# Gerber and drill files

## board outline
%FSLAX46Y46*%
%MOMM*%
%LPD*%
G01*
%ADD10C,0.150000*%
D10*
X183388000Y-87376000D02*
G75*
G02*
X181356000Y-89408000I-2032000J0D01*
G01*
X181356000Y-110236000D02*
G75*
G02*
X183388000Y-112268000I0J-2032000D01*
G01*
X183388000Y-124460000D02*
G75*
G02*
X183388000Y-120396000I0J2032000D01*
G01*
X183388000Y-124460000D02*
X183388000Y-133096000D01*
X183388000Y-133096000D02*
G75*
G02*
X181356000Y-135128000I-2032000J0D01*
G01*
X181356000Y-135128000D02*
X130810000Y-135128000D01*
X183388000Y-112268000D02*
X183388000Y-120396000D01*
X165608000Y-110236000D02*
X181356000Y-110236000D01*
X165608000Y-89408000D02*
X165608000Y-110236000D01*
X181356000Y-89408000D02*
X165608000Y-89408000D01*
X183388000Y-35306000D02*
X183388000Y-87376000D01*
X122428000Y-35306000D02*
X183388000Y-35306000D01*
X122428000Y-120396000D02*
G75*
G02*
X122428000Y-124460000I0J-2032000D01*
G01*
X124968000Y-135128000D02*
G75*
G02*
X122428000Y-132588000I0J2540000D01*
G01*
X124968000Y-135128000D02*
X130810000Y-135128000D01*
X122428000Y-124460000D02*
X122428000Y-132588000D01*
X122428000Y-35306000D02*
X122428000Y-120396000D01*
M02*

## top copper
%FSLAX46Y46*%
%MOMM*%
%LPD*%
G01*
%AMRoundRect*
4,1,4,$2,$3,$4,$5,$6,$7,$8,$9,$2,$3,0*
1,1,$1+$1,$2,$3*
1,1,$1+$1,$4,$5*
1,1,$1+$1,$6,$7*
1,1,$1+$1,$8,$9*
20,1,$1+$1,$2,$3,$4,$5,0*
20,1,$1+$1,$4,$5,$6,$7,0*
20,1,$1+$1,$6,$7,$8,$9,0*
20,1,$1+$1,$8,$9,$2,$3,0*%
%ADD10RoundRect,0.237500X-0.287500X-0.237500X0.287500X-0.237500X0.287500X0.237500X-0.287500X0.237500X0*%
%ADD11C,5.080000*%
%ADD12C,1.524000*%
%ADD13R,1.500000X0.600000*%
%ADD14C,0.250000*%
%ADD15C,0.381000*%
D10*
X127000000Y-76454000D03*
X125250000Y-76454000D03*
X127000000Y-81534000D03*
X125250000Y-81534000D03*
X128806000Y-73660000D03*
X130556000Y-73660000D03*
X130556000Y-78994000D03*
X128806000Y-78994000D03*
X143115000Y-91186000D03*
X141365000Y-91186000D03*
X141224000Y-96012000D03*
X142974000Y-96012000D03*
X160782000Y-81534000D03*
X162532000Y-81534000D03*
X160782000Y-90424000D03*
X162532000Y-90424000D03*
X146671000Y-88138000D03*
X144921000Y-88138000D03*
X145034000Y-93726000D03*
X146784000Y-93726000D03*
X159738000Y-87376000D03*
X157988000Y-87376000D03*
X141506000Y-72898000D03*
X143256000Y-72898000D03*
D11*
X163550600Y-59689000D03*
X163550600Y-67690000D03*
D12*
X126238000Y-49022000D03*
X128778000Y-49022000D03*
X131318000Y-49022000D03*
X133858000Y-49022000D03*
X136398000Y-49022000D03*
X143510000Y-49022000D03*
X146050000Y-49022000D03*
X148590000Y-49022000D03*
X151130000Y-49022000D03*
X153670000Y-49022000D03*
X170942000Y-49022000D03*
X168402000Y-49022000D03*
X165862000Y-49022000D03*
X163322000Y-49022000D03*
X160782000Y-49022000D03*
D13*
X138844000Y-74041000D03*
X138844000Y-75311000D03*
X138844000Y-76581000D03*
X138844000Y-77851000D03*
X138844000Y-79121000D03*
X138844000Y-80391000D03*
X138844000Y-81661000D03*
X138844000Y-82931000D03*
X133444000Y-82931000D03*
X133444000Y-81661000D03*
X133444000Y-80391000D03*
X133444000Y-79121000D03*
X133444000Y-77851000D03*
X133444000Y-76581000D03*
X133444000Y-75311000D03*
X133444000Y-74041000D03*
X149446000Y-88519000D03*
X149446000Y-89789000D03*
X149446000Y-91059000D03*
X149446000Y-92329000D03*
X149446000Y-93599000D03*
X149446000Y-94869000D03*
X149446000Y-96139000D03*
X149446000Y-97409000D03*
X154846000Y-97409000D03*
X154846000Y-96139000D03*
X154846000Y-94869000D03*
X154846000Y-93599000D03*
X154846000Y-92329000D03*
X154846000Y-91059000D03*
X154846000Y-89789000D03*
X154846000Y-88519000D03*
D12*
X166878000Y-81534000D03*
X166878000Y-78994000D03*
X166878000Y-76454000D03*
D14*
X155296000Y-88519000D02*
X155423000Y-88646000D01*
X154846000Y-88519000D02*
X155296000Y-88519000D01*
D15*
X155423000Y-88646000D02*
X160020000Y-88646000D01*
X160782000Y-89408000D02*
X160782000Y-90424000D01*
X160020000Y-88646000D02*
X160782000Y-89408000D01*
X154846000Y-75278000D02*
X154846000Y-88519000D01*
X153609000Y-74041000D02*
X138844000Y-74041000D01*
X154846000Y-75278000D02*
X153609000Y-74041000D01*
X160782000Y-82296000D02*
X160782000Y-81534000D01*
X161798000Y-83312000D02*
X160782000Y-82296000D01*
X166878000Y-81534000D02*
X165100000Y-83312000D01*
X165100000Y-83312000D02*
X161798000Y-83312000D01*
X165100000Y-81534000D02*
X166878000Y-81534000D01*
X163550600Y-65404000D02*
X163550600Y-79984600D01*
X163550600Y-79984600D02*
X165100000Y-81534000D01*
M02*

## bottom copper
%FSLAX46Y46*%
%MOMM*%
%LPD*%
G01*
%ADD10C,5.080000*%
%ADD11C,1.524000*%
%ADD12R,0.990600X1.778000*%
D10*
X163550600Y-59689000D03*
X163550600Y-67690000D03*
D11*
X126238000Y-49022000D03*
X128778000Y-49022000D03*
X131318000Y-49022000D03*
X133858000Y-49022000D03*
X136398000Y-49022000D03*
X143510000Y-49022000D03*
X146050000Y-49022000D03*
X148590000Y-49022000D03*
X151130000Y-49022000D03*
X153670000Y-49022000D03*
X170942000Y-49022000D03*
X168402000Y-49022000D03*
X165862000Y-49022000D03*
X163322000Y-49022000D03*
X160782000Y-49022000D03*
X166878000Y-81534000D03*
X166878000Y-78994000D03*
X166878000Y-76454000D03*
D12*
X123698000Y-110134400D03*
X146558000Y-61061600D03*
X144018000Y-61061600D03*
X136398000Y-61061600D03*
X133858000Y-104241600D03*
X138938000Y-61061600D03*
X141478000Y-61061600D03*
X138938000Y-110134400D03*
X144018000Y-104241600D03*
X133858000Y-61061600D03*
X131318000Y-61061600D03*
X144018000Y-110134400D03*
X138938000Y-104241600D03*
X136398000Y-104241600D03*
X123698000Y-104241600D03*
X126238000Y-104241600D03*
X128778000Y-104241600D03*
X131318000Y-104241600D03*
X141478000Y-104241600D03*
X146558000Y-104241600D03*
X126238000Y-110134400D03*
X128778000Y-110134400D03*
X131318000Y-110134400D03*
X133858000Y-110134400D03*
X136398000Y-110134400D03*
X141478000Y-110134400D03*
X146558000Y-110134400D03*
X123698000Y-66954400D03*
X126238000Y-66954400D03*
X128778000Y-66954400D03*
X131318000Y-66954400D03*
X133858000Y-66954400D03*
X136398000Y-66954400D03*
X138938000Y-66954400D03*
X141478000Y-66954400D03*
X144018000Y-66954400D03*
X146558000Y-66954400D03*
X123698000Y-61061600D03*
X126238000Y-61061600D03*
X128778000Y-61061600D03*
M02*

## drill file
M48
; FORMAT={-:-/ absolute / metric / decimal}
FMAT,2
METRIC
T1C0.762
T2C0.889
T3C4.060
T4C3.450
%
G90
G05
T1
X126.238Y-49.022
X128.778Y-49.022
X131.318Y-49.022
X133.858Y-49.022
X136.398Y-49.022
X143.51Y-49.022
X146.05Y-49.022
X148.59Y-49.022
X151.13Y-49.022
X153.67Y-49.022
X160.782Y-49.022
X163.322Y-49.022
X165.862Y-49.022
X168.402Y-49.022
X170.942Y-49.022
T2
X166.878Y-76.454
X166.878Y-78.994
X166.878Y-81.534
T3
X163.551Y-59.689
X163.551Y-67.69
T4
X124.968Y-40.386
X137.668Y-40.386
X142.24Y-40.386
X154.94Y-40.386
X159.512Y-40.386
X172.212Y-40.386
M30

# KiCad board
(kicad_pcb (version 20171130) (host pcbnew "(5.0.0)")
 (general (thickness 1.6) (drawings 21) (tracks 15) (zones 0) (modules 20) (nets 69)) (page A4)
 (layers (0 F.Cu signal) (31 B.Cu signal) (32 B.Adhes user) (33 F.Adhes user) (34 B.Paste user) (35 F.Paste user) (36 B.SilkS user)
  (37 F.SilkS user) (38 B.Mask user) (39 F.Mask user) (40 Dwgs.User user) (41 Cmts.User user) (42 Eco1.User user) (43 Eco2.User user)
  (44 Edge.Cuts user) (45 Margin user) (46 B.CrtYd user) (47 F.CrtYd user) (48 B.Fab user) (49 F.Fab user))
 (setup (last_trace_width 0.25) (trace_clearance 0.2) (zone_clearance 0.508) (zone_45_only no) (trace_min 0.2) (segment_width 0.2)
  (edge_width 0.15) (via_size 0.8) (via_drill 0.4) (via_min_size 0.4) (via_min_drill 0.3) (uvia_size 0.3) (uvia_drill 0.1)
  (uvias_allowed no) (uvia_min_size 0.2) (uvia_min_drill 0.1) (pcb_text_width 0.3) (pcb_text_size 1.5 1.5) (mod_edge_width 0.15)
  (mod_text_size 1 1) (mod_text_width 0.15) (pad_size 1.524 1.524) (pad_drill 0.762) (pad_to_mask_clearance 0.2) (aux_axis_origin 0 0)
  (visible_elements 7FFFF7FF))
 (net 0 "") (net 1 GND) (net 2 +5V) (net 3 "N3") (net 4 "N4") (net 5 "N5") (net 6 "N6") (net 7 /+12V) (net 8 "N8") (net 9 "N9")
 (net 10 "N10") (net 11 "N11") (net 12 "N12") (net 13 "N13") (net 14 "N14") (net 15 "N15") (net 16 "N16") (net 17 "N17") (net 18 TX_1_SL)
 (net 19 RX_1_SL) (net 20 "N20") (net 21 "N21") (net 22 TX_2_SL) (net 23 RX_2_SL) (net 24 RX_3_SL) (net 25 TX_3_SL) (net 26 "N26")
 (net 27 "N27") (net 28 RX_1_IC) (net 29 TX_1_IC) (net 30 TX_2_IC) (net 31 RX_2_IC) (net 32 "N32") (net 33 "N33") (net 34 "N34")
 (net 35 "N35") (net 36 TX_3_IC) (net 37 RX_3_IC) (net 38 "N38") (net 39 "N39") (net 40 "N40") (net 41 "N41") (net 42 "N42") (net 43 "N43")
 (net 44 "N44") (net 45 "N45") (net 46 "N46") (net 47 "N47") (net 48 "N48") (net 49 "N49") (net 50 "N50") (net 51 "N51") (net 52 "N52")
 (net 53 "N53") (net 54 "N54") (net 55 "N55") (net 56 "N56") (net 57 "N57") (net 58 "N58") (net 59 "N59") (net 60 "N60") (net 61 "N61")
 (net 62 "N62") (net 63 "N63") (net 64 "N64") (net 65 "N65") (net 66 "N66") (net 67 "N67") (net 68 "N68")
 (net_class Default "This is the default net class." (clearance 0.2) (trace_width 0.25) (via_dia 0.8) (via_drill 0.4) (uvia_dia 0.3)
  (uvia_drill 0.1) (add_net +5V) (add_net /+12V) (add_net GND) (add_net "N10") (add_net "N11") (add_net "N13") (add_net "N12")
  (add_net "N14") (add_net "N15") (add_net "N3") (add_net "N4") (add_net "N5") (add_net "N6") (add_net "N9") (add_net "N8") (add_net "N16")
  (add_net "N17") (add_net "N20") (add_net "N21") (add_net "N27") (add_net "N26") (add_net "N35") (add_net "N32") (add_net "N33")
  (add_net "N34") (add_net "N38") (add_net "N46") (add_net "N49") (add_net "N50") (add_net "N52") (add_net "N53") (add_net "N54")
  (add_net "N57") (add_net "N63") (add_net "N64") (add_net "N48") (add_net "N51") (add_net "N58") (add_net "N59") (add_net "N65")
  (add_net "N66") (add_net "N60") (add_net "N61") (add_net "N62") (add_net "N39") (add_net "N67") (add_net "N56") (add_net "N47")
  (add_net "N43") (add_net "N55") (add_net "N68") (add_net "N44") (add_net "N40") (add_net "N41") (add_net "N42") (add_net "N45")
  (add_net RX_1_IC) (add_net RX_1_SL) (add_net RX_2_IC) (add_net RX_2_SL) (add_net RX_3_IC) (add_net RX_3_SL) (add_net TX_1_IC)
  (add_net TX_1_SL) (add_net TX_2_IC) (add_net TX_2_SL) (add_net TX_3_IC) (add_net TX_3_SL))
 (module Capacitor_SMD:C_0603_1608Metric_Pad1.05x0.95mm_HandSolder (layer F.Cu) (at 126.125 76.454)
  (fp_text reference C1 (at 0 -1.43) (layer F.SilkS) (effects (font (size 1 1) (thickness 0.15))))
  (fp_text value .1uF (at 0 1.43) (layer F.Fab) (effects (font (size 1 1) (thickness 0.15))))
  (pad 2 smd roundrect (at 0.875 0) (size 1.05 0.95) (layers F.Cu F.Paste F.Mask) (roundrect_rratio 0.25) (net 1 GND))
  (pad 1 smd roundrect (at -0.875 0) (size 1.05 0.95) (layers F.Cu F.Paste F.Mask) (roundrect_rratio 0.25) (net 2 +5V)))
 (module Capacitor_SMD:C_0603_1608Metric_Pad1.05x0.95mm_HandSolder (layer F.Cu) (at 126.125 81.534)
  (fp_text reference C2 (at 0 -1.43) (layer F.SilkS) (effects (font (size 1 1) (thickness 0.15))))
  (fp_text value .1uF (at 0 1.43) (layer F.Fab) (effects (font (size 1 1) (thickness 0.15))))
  (pad 2 smd roundrect (at 0.875 0) (size 1.05 0.95) (layers F.Cu F.Paste F.Mask) (roundrect_rratio 0.25) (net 1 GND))
  (pad 1 smd roundrect (at -0.875 0) (size 1.05 0.95) (layers F.Cu F.Paste F.Mask) (roundrect_rratio 0.25) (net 2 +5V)))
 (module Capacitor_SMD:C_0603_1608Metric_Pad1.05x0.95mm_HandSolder (layer F.Cu) (at 129.681 73.66)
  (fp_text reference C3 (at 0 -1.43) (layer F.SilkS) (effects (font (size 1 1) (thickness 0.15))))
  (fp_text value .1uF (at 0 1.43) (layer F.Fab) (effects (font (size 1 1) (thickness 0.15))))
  (pad 1 smd roundrect (at -0.875 0) (size 1.05 0.95) (layers F.Cu F.Paste F.Mask) (roundrect_rratio 0.25) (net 1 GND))
  (pad 2 smd roundrect (at 0.875 0) (size 1.05 0.95) (layers F.Cu F.Paste F.Mask) (roundrect_rratio 0.25) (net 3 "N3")))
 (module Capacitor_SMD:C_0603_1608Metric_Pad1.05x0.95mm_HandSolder (layer F.Cu) (at 129.681 78.994)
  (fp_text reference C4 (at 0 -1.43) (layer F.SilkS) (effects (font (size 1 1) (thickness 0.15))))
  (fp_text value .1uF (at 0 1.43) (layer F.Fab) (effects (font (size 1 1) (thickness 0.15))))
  (pad 2 smd roundrect (at 0.875 0) (size 1.05 0.95) (layers F.Cu F.Paste F.Mask) (roundrect_rratio 0.25) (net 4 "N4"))
  (pad 1 smd roundrect (at -0.875 0) (size 1.05 0.95) (layers F.Cu F.Paste F.Mask) (roundrect_rratio 0.25) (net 1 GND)))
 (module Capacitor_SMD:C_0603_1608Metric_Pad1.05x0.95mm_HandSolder (layer F.Cu) (at 142.24 91.186)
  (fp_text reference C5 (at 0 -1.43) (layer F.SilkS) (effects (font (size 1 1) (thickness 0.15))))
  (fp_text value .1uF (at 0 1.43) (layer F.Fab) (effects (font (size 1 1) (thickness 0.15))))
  (pad 2 smd roundrect (at 0.875 0) (size 1.05 0.95) (layers F.Cu F.Paste F.Mask) (roundrect_rratio 0.25) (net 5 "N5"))
  (pad 1 smd roundrect (at -0.875 0) (size 1.05 0.95) (layers F.Cu F.Paste F.Mask) (roundrect_rratio 0.25) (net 1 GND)))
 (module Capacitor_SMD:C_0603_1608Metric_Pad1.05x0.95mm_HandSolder (layer F.Cu) (at 142.099 96.012)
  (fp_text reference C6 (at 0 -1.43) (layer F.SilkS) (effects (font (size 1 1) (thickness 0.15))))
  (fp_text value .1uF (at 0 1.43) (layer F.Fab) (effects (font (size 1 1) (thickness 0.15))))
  (pad 1 smd roundrect (at -0.875 0) (size 1.05 0.95) (layers F.Cu F.Paste F.Mask) (roundrect_rratio 0.25) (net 1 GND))
  (pad 2 smd roundrect (at 0.875 0) (size 1.05 0.95) (layers F.Cu F.Paste F.Mask) (roundrect_rratio 0.25) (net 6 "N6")))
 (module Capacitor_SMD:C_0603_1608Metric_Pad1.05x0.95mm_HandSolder (layer F.Cu) (at 161.657 81.534)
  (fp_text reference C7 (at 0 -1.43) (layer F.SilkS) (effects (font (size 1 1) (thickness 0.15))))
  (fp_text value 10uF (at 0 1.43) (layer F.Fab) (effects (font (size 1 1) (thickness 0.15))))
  (pad 1 smd roundrect (at -0.875 0) (size 1.05 0.95) (layers F.Cu F.Paste F.Mask) (roundrect_rratio 0.25) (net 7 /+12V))
  (pad 2 smd roundrect (at 0.875 0) (size 1.05 0.95) (layers F.Cu F.Paste F.Mask) (roundrect_rratio 0.25) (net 1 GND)))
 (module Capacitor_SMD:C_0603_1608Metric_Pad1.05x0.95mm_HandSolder (layer F.Cu) (at 161.657 90.424)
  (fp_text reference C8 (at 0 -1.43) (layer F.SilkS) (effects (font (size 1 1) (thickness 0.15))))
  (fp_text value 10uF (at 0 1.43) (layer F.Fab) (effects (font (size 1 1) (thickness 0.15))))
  (pad 1 smd roundrect (at -0.875 0) (size 1.05 0.95) (layers F.Cu F.Paste F.Mask) (roundrect_rratio 0.25) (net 2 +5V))
  (pad 2 smd roundrect (at 0.875 0) (size 1.05 0.95) (layers F.Cu F.Paste F.Mask) (roundrect_rratio 0.25) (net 1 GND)))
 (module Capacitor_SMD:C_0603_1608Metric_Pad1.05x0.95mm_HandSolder (layer F.Cu) (at 145.796 88.138)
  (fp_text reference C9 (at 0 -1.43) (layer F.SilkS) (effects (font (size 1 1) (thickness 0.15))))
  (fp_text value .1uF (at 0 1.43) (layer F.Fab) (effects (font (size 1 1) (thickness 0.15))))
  (pad 2 smd roundrect (at 0.875 0) (size 1.05 0.95) (layers F.Cu F.Paste F.Mask) (roundrect_rratio 0.25) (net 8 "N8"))
  (pad 1 smd roundrect (at -0.875 0) (size 1.05 0.95) (layers F.Cu F.Paste F.Mask) (roundrect_rratio 0.25) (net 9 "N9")))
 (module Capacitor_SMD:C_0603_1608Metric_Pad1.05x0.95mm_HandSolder (layer F.Cu) (at 145.909 93.726)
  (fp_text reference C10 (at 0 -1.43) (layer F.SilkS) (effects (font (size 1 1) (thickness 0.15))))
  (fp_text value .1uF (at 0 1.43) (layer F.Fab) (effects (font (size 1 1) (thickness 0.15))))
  (pad 1 smd roundrect (at -0.875 0) (size 1.05 0.95) (layers F.Cu F.Paste F.Mask) (roundrect_rratio 0.25) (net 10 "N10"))
  (pad 2 smd roundrect (at 0.875 0) (size 1.05 0.95) (layers F.Cu F.Paste F.Mask) (roundrect_rratio 0.25) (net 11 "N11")))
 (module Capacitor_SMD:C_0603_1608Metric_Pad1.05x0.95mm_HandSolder (layer F.Cu) (at 158.863 87.376)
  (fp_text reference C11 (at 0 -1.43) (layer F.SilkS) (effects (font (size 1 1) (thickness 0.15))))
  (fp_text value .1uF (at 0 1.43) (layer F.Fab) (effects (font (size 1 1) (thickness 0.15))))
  (pad 2 smd roundrect (at 0.875 0) (size 1.05 0.95) (layers F.Cu F.Paste F.Mask) (roundrect_rratio 0.25) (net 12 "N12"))
  (pad 1 smd roundrect (at -0.875 0) (size 1.05 0.95) (layers F.Cu F.Paste F.Mask) (roundrect_rratio 0.25) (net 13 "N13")))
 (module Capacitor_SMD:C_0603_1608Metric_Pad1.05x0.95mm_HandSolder (layer F.Cu) (at 142.381 72.898)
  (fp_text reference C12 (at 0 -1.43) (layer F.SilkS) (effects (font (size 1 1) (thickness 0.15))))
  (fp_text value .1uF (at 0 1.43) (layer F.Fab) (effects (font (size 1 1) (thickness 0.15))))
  (pad 1 smd roundrect (at -0.875 0) (size 1.05 0.95) (layers F.Cu F.Paste F.Mask) (roundrect_rratio 0.25) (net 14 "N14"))
  (pad 2 smd roundrect (at 0.875 0) (size 1.05 0.95) (layers F.Cu F.Paste F.Mask) (roundrect_rratio 0.25) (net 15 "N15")))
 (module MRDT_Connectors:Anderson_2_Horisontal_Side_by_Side (layer F.Cu) (at 167.132 55.626 180)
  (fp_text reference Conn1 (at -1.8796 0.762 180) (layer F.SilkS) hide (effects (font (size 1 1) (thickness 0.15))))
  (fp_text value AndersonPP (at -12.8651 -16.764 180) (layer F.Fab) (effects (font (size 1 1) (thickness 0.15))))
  (pad 1 thru_hole circle (at 3.5814 -4.063 180) (size 5.08 5.08) (drill 4.06) (layers *.Cu *.Mask F.Paste) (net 1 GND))
  (pad 2 thru_hole circle (at 3.5814 -12.064 180) (size 5.08 5.08) (drill 4.06) (layers *.Cu *.Mask F.Paste) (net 7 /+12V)))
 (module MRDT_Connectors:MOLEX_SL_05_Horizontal (layer F.Cu) (at 131.318 49.022)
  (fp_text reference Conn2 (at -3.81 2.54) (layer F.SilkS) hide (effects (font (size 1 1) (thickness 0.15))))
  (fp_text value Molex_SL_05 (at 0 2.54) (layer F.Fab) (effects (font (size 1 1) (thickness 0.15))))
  (pad 1 thru_hole circle (at -5.08 0) (size 1.524 1.524) (drill 0.762) (layers *.Cu *.Mask) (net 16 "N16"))
  (pad 2 thru_hole circle (at -2.54 0) (size 1.524 1.524) (drill 0.762) (layers *.Cu *.Mask) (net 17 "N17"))
  (pad 3 thru_hole circle (at 0 0) (size 1.524 1.524) (drill 0.762) (layers *.Cu *.Mask) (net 1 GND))
  (pad 4 thru_hole circle (at 2.54 0) (size 1.524 1.524) (drill 0.762) (layers *.Cu *.Mask) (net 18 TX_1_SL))
  (pad 5 thru_hole circle (at 5.08 0) (size 1.524 1.524) (drill 0.762) (layers *.Cu *.Mask) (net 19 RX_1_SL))
  (pad "" np_thru_hole circle (at -6.35 -8.636) (size 3.45 3.45) (drill 3.45) (layers *.Cu *.Mask))
  (pad "" np_thru_hole circle (at 6.35 -8.636) (size 3.45 3.45) (drill 3.45) (layers *.Cu *.Mask)))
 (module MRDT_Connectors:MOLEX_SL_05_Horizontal (layer F.Cu) (at 148.59 49.022)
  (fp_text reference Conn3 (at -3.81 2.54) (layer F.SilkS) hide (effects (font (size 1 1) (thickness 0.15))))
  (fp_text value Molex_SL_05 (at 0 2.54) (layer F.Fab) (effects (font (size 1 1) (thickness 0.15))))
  (pad 1 thru_hole circle (at -5.08 0) (size 1.524 1.524) (drill 0.762) (layers *.Cu *.Mask) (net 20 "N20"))
  (pad 2 thru_hole circle (at -2.54 0) (size 1.524 1.524) (drill 0.762) (layers *.Cu *.Mask) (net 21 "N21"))
  (pad 3 thru_hole circle (at 0 0) (size 1.524 1.524) (drill 0.762) (layers *.Cu *.Mask) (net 1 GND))
  (pad 4 thru_hole circle (at 2.54 0) (size 1.524 1.524) (drill 0.762) (layers *.Cu *.Mask) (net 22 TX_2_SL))
  (pad 5 thru_hole circle (at 5.08 0) (size 1.524 1.524) (drill 0.762) (layers *.Cu *.Mask) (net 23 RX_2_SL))
  (pad "" np_thru_hole circle (at -6.35 -8.636) (size 3.45 3.45) (drill 3.45) (layers *.Cu *.Mask))
  (pad "" np_thru_hole circle (at 6.35 -8.636) (size 3.45 3.45) (drill 3.45) (layers *.Cu *.Mask)))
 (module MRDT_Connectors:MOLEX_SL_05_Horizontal (layer F.Cu) (at 165.862 49.022)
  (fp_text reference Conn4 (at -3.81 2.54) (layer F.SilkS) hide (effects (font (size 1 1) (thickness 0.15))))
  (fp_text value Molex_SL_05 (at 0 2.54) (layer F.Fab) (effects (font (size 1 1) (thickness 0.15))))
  (pad "" np_thru_hole circle (at 6.35 -8.636) (size 3.45 3.45) (drill 3.45) (layers *.Cu *.Mask))
  (pad "" np_thru_hole circle (at -6.35 -8.636) (size 3.45 3.45) (drill 3.45) (layers *.Cu *.Mask))
  (pad 5 thru_hole circle (at 5.08 0) (size 1.524 1.524) (drill 0.762) (layers *.Cu *.Mask) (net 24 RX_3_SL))
  (pad 4 thru_hole circle (at 2.54 0) (size 1.524 1.524) (drill 0.762) (layers *.Cu *.Mask) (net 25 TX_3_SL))
  (pad 3 thru_hole circle (at 0 0) (size 1.524 1.524) (drill 0.762) (layers *.Cu *.Mask) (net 1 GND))
  (pad 2 thru_hole circle (at -2.54 0) (size 1.524 1.524) (drill 0.762) (layers *.Cu *.Mask) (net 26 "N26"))
  (pad 1 thru_hole circle (at -5.08 0) (size 1.524 1.524) (drill 0.762) (layers *.Cu *.Mask) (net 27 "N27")))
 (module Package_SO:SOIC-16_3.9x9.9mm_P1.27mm (layer F.Cu) (at 136.144 78.486)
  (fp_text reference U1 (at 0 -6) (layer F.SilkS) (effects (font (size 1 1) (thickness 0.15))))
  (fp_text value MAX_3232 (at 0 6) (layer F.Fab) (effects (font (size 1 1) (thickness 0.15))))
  (pad 16 smd rect (at 2.7 -4.445) (size 1.5 0.6) (layers F.Cu F.Paste F.Mask) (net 2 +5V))
  (pad 15 smd rect (at 2.7 -3.175) (size 1.5 0.6) (layers F.Cu F.Paste F.Mask) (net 1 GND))
  (pad 14 smd rect (at 2.7 -1.905) (size 1.5 0.6) (layers F.Cu F.Paste F.Mask) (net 18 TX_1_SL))
  (pad 13 smd rect (at 2.7 -0.635) (size 1.5 0.6) (layers F.Cu F.Paste F.Mask) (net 19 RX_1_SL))
  (pad 12 smd rect (at 2.7 0.635) (size 1.5 0.6) (layers F.Cu F.Paste F.Mask) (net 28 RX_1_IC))
  (pad 11 smd rect (at 2.7 1.905) (size 1.5 0.6) (layers F.Cu F.Paste F.Mask) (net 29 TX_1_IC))
  (pad 10 smd rect (at 2.7 3.175) (size 1.5 0.6) (layers F.Cu F.Paste F.Mask) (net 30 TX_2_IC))
  (pad 9 smd rect (at 2.7 4.445) (size 1.5 0.6) (layers F.Cu F.Paste F.Mask) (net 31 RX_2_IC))
  (pad 8 smd rect (at -2.7 4.445) (size 1.5 0.6) (layers F.Cu F.Paste F.Mask) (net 23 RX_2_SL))
  (pad 7 smd rect (at -2.7 3.175) (size 1.5 0.6) (layers F.Cu F.Paste F.Mask) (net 22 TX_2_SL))
  (pad 6 smd rect (at -2.7 1.905) (size 1.5 0.6) (layers F.Cu F.Paste F.Mask) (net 4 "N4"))
  (pad 5 smd rect (at -2.7 0.635) (size 1.5 0.6) (layers F.Cu F.Paste F.Mask) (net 11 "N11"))
  (pad 4 smd rect (at -2.7 -0.635) (size 1.5 0.6) (layers F.Cu F.Paste F.Mask) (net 10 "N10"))
  (pad 3 smd rect (at -2.7 -1.905) (size 1.5 0.6) (layers F.Cu F.Paste F.Mask) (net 8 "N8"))
  (pad 2 smd rect (at -2.7 -3.175) (size 1.5 0.6) (layers F.Cu F.Paste F.Mask) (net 3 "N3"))
  (pad 1 smd rect (at -2.7 -4.445) (size 1.5 0.6) (layers F.Cu F.Paste F.Mask) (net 9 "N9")))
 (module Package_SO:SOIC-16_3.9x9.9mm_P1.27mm (layer F.Cu) (at 152.146 92.964)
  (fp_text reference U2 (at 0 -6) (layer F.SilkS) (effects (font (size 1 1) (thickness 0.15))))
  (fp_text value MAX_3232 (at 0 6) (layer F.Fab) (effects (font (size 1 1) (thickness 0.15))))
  (pad 1 smd rect (at -2.7 -4.445) (size 1.5 0.6) (layers F.Cu F.Paste F.Mask) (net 13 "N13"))
  (pad 2 smd rect (at -2.7 -3.175) (size 1.5 0.6) (layers F.Cu F.Paste F.Mask) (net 5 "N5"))
  (pad 3 smd rect (at -2.7 -1.905) (size 1.5 0.6) (layers F.Cu F.Paste F.Mask) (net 12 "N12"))
  (pad 4 smd rect (at -2.7 -0.635) (size 1.5 0.6) (layers F.Cu F.Paste F.Mask) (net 14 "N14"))
  (pad 5 smd rect (at -2.7 0.635) (size 1.5 0.6) (layers F.Cu F.Paste F.Mask) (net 15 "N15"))
  (pad 6 smd rect (at -2.7 1.905) (size 1.5 0.6) (layers F.Cu F.Paste F.Mask) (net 6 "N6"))
  (pad 7 smd rect (at -2.7 3.175) (size 1.5 0.6) (layers F.Cu F.Paste F.Mask) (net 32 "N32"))
  (pad 8 smd rect (at -2.7 4.445) (size 1.5 0.6) (layers F.Cu F.Paste F.Mask) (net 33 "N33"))
  (pad 9 smd rect (at 2.7 4.445) (size 1.5 0.6) (layers F.Cu F.Paste F.Mask) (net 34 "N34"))
  (pad 10 smd rect (at 2.7 3.175) (size 1.5 0.6) (layers F.Cu F.Paste F.Mask) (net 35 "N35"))
  (pad 11 smd rect (at 2.7 1.905) (size 1.5 0.6) (layers F.Cu F.Paste F.Mask) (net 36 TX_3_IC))
  (pad 12 smd rect (at 2.7 0.635) (size 1.5 0.6) (layers F.Cu F.Paste F.Mask) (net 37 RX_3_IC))
  (pad 13 smd rect (at 2.7 -0.635) (size 1.5 0.6) (layers F.Cu F.Paste F.Mask) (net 24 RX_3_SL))
  (pad 14 smd rect (at 2.7 -1.905) (size 1.5 0.6) (layers F.Cu F.Paste F.Mask) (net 25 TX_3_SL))
  (pad 15 smd rect (at 2.7 -3.175) (size 1.5 0.6) (layers F.Cu F.Paste F.Mask) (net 1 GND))
  (pad 16 smd rect (at 2.7 -4.445) (size 1.5 0.6) (layers F.Cu F.Paste F.Mask) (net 2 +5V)))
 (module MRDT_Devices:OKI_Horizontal (layer F.Cu) (at 165.608 84.074 90)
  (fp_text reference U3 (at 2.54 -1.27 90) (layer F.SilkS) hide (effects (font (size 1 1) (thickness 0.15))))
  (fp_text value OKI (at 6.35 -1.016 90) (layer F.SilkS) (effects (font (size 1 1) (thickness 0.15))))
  (pad 1 thru_hole circle (at 2.54 1.27 90) (size 1.524 1.524) (drill 0.889) (layers *.Cu *.Mask) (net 7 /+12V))
  (pad 2 thru_hole circle (at 5.08 1.27 90) (size 1.524 1.524) (drill 0.889) (layers *.Cu *.Mask) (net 1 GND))
  (pad 3 thru_hole circle (at 7.62 1.27 90) (size 1.524 1.524) (drill 0.889) (layers *.Cu *.Mask) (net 2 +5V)))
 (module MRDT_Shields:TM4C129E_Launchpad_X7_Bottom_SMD (layer F.Cu) (at 122.428 109.728)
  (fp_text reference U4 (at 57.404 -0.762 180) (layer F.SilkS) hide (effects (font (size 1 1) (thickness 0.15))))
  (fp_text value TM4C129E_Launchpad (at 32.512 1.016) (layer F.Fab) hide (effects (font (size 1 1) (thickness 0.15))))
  (pad +3V3 smd rect (at 1.27 0.4064 180) (size 0.9906 1.778) (layers B.Cu B.Paste B.Mask) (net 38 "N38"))
  (pad PM6 smd rect (at 24.13 -48.6664 180) (size 0.9906 1.778) (layers B.Cu B.Paste B.Mask) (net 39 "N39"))
  (pad PQ1 smd rect (at 21.59 -48.6664 180) (size 0.9906 1.778) (layers B.Cu B.Paste B.Mask) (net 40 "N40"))
  (pad PQ2 smd rect (at 13.97 -48.6664 180) (size 0.9906 1.778) (layers B.Cu B.Paste B.Mask) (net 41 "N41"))
  (pad PK0 smd rect (at 11.43 -5.4864 180) (size 0.9906 1.778) (layers B.Cu B.Paste B.Mask) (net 28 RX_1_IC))
  (pad PQ3 smd rect (at 16.51 -48.6664 180) (size 0.9906 1.778) (layers B.Cu B.Paste B.Mask) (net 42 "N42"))
  (pad PP3 smd rect (at 19.05 -48.6664 180) (size 0.9906 1.778) (layers B.Cu B.Paste B.Mask) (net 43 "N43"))
  (pad PQ0 smd rect (at 16.51 0.4064 180) (size 0.9906 1.778) (layers B.Cu B.Paste B.Mask) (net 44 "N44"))
  (pad PA4 smd rect (at 21.59 -5.4864 180) (size 0.9906 1.778) (layers B.Cu B.Paste B.Mask) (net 37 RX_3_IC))
  (pad Rese smd rect (at 11.43 -48.6664 180) (size 0.9906 1.778) (layers B.Cu B.Paste B.Mask) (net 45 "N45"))
  (pad PA7 smd rect (at 8.89 -48.6664 180) (size 0.9906 1.778) (layers B.Cu B.Paste B.Mask) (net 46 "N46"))
  (pad PN5 smd rect (at 21.59 0.4064 180) (size 0.9906 1.778) (layers B.Cu B.Paste B.Mask) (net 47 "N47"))
  (pad PK2 smd rect (at 16.51 -5.4864 180) (size 0.9906 1.778) (layers B.Cu B.Paste B.Mask) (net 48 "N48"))
  (pad PK1 smd rect (at 13.97 -5.4864 180) (size 0.9906 1.778) (layers B.Cu B.Paste B.Mask) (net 29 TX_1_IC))
  (pad +5V smd rect (at 1.27 -5.4864 180) (size 0.9906 1.778) (layers B.Cu B.Paste B.Mask) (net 2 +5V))
  (pad GND smd rect (at 3.81 -5.4864 180) (size 0.9906 1.778) (layers B.Cu B.Paste B.Mask) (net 1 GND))
  (pad PB4 smd rect (at 6.35 -5.4864 180) (size 0.9906 1.778) (layers B.Cu B.Paste B.Mask) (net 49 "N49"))
  (pad PB5 smd rect (at 8.89 -5.4864 180) (size 0.9906 1.778) (layers B.Cu B.Paste B.Mask) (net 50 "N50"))
  (pad PK3 smd rect (at 19.05 -5.4864 180) (size 0.9906 1.778) (layers B.Cu B.Paste B.Mask) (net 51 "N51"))
  (pad PA5 smd rect (at 24.13 -5.4864 180) (size 0.9906 1.778) (layers B.Cu B.Paste B.Mask) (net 36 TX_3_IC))
  (pad PD2 smd rect (at 3.81 0.4064 180) (size 0.9906 1.778) (layers B.Cu B.Paste B.Mask) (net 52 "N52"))
  (pad PP0 smd rect (at 6.35 0.4064 180) (size 0.9906 1.778) (layers B.Cu B.Paste B.Mask) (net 31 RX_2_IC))
  (pad PP1 smd rect (at 8.89 0.4064 180) (size 0.9906 1.778) (layers B.Cu B.Paste B.Mask) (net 30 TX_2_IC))
  (pad PD4 smd rect (at 11.43 0.4064 180) (size 0.9906 1.778) (layers B.Cu B.Paste B.Mask) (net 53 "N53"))
  (pad PD5 smd rect (at 13.97 0.4064 180) (size 0.9906 1.778) (layers B.Cu B.Paste B.Mask) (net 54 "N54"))
  (pad PP4 smd rect (at 19.05 0.4064 180) (size 0.9906 1.778) (layers B.Cu B.Paste B.Mask) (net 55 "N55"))
  (pad PN4 smd rect (at 24.13 0.4064 180) (size 0.9906 1.778) (layers B.Cu B.Paste B.Mask) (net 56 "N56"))
  (pad PG1 smd rect (at 1.27 -42.7736 180) (size 0.9906 1.778) (layers B.Cu B.Paste B.Mask) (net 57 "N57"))
  (pad PK4 smd rect (at 3.81 -42.7736 180) (size 0.9906 1.778) (layers B.Cu B.Paste B.Mask) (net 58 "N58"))
  (pad PK5 smd rect (at 6.35 -42.7736 180) (size 0.9906 1.778) (layers B.Cu B.Paste B.Mask) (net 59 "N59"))
  (pad PM0 smd rect (at 8.89 -42.7736 180) (size 0.9906 1.778) (layers B.Cu B.Paste B.Mask) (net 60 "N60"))
  (pad PM1 smd rect (at 11.43 -42.7736 180) (size 0.9906 1.778) (layers B.Cu B.Paste B.Mask) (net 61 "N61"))
  (pad PM2 smd rect (at 13.97 -42.7736 180) (size 0.9906 1.778) (layers B.Cu B.Paste B.Mask) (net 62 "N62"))
  (pad PH0 smd rect (at 16.51 -42.7736 180) (size 0.9906 1.778) (layers B.Cu B.Paste B.Mask) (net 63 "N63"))
  (pad PH1 smd rect (at 19.05 -42.7736 180) (size 0.9906 1.778) (layers B.Cu B.Paste B.Mask) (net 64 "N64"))
  (pad PK6 smd rect (at 21.59 -42.7736 180) (size 0.9906 1.778) (layers B.Cu B.Paste B.Mask) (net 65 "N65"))
  (pad PK7 smd rect (at 24.13 -42.7736 180) (size 0.9906 1.778) (layers B.Cu B.Paste B.Mask) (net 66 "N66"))
  (pad GND smd rect (at 1.27 -48.6664 180) (size 0.9906 1.778) (layers B.Cu B.Paste B.Mask) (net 1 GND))
  (pad PM7 smd rect (at 3.81 -48.6664 180) (size 0.9906 1.778) (layers B.Cu B.Paste B.Mask) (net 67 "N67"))
  (pad PP5 smd rect (at 6.35 -48.6664 180) (size 0.9906 1.778) (layers B.Cu B.Paste B.Mask) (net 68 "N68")))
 (gr_arc (start 181.356 87.376) (end 181.356 89.408) (angle -90) (layer Edge.Cuts) (width 0.15))
 (gr_arc (start 181.356 112.268) (end 183.388 112.268) (angle -90) (layer Edge.Cuts) (width 0.15))
 (gr_arc (start 183.388 122.428) (end 183.388 120.396) (angle -180) (layer Edge.Cuts) (width 0.15))
 (gr_line (start 183.388 124.46) (end 183.388 133.096) (layer Edge.Cuts) (width 0.15))
 (gr_arc (start 181.356 133.096) (end 181.356 135.128) (angle -90) (layer Edge.Cuts) (width 0.15))
 (gr_line (start 181.356 135.128) (end 130.81 135.128) (layer Edge.Cuts) (width 0.15))
 (gr_line (start 183.388 112.268) (end 183.388 120.396) (layer Edge.Cuts) (width 0.15))
 (gr_line (start 165.608 110.236) (end 181.356 110.236) (layer Edge.Cuts) (width 0.15))
 (gr_line (start 165.608 89.408) (end 165.608 110.236) (layer Edge.Cuts) (width 0.15))
 (gr_line (start 181.356 89.408) (end 165.608 89.408) (layer Edge.Cuts) (width 0.15))
 (gr_line (start 183.388 35.306) (end 183.388 87.376) (layer Edge.Cuts) (width 0.15))
 (gr_line (start 122.428 35.306) (end 183.388 35.306) (layer Edge.Cuts) (width 0.15))
 (gr_arc (start 122.428 122.428) (end 122.428 124.46) (angle -180) (layer Edge.Cuts) (width 0.15))
 (gr_arc (start 124.968 132.588) (end 122.428 132.588) (angle -90) (layer Edge.Cuts) (width 0.15))
 (gr_line (start 124.968 135.128) (end 130.81 135.128) (layer Edge.Cuts) (width 0.15))
 (gr_line (start 122.428 124.46) (end 122.428 132.588) (layer Edge.Cuts) (width 0.15))
 (gr_line (start 122.428 35.306) (end 122.428 120.396) (layer Edge.Cuts) (width 0.15))
 (segment (start 155.296 88.519) (end 155.423 88.646) (width 0.25) (layer F.Cu) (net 2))
 (segment (start 154.846 88.519) (end 155.296 88.519) (width 0.25) (layer F.Cu) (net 2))
 (segment (start 155.423 88.646) (end 160.02 88.646) (width 0.381) (layer F.Cu) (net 2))
 (segment (start 160.782 89.408) (end 160.782 90.424) (width 0.381) (layer F.Cu) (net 2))
 (segment (start 160.02 88.646) (end 160.782 89.408) (width 0.381) (layer F.Cu) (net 2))
 (segment (start 154.846 75.278) (end 154.846 88.519) (width 0.381) (layer F.Cu) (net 2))
 (segment (start 153.609 74.041) (end 138.844 74.041) (width 0.381) (layer F.Cu) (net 2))
 (segment (start 154.846 75.278) (end 153.609 74.041) (width 0.381) (layer F.Cu) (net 2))
 (segment (start 160.782 82.296) (end 160.782 81.534) (width 0.381) (layer F.Cu) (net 7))
 (segment (start 161.798 83.312) (end 160.782 82.296) (width 0.381) (layer F.Cu) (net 7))
 (segment (start 166.878 81.534) (end 165.1 83.312) (width 0.381) (layer F.Cu) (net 7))
 (segment (start 165.1 83.312) (end 161.798 83.312) (width 0.381) (layer F.Cu) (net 7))
 (segment (start 165.1 81.534) (end 166.878 81.534) (width 0.381) (layer F.Cu) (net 7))
 (segment (start 163.5506 65.404) (end 163.5506 79.9846) (width 0.381) (layer F.Cu) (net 7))
 (segment (start 163.5506 79.9846) (end 165.1 81.534) (width 0.381) (layer F.Cu) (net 7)))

